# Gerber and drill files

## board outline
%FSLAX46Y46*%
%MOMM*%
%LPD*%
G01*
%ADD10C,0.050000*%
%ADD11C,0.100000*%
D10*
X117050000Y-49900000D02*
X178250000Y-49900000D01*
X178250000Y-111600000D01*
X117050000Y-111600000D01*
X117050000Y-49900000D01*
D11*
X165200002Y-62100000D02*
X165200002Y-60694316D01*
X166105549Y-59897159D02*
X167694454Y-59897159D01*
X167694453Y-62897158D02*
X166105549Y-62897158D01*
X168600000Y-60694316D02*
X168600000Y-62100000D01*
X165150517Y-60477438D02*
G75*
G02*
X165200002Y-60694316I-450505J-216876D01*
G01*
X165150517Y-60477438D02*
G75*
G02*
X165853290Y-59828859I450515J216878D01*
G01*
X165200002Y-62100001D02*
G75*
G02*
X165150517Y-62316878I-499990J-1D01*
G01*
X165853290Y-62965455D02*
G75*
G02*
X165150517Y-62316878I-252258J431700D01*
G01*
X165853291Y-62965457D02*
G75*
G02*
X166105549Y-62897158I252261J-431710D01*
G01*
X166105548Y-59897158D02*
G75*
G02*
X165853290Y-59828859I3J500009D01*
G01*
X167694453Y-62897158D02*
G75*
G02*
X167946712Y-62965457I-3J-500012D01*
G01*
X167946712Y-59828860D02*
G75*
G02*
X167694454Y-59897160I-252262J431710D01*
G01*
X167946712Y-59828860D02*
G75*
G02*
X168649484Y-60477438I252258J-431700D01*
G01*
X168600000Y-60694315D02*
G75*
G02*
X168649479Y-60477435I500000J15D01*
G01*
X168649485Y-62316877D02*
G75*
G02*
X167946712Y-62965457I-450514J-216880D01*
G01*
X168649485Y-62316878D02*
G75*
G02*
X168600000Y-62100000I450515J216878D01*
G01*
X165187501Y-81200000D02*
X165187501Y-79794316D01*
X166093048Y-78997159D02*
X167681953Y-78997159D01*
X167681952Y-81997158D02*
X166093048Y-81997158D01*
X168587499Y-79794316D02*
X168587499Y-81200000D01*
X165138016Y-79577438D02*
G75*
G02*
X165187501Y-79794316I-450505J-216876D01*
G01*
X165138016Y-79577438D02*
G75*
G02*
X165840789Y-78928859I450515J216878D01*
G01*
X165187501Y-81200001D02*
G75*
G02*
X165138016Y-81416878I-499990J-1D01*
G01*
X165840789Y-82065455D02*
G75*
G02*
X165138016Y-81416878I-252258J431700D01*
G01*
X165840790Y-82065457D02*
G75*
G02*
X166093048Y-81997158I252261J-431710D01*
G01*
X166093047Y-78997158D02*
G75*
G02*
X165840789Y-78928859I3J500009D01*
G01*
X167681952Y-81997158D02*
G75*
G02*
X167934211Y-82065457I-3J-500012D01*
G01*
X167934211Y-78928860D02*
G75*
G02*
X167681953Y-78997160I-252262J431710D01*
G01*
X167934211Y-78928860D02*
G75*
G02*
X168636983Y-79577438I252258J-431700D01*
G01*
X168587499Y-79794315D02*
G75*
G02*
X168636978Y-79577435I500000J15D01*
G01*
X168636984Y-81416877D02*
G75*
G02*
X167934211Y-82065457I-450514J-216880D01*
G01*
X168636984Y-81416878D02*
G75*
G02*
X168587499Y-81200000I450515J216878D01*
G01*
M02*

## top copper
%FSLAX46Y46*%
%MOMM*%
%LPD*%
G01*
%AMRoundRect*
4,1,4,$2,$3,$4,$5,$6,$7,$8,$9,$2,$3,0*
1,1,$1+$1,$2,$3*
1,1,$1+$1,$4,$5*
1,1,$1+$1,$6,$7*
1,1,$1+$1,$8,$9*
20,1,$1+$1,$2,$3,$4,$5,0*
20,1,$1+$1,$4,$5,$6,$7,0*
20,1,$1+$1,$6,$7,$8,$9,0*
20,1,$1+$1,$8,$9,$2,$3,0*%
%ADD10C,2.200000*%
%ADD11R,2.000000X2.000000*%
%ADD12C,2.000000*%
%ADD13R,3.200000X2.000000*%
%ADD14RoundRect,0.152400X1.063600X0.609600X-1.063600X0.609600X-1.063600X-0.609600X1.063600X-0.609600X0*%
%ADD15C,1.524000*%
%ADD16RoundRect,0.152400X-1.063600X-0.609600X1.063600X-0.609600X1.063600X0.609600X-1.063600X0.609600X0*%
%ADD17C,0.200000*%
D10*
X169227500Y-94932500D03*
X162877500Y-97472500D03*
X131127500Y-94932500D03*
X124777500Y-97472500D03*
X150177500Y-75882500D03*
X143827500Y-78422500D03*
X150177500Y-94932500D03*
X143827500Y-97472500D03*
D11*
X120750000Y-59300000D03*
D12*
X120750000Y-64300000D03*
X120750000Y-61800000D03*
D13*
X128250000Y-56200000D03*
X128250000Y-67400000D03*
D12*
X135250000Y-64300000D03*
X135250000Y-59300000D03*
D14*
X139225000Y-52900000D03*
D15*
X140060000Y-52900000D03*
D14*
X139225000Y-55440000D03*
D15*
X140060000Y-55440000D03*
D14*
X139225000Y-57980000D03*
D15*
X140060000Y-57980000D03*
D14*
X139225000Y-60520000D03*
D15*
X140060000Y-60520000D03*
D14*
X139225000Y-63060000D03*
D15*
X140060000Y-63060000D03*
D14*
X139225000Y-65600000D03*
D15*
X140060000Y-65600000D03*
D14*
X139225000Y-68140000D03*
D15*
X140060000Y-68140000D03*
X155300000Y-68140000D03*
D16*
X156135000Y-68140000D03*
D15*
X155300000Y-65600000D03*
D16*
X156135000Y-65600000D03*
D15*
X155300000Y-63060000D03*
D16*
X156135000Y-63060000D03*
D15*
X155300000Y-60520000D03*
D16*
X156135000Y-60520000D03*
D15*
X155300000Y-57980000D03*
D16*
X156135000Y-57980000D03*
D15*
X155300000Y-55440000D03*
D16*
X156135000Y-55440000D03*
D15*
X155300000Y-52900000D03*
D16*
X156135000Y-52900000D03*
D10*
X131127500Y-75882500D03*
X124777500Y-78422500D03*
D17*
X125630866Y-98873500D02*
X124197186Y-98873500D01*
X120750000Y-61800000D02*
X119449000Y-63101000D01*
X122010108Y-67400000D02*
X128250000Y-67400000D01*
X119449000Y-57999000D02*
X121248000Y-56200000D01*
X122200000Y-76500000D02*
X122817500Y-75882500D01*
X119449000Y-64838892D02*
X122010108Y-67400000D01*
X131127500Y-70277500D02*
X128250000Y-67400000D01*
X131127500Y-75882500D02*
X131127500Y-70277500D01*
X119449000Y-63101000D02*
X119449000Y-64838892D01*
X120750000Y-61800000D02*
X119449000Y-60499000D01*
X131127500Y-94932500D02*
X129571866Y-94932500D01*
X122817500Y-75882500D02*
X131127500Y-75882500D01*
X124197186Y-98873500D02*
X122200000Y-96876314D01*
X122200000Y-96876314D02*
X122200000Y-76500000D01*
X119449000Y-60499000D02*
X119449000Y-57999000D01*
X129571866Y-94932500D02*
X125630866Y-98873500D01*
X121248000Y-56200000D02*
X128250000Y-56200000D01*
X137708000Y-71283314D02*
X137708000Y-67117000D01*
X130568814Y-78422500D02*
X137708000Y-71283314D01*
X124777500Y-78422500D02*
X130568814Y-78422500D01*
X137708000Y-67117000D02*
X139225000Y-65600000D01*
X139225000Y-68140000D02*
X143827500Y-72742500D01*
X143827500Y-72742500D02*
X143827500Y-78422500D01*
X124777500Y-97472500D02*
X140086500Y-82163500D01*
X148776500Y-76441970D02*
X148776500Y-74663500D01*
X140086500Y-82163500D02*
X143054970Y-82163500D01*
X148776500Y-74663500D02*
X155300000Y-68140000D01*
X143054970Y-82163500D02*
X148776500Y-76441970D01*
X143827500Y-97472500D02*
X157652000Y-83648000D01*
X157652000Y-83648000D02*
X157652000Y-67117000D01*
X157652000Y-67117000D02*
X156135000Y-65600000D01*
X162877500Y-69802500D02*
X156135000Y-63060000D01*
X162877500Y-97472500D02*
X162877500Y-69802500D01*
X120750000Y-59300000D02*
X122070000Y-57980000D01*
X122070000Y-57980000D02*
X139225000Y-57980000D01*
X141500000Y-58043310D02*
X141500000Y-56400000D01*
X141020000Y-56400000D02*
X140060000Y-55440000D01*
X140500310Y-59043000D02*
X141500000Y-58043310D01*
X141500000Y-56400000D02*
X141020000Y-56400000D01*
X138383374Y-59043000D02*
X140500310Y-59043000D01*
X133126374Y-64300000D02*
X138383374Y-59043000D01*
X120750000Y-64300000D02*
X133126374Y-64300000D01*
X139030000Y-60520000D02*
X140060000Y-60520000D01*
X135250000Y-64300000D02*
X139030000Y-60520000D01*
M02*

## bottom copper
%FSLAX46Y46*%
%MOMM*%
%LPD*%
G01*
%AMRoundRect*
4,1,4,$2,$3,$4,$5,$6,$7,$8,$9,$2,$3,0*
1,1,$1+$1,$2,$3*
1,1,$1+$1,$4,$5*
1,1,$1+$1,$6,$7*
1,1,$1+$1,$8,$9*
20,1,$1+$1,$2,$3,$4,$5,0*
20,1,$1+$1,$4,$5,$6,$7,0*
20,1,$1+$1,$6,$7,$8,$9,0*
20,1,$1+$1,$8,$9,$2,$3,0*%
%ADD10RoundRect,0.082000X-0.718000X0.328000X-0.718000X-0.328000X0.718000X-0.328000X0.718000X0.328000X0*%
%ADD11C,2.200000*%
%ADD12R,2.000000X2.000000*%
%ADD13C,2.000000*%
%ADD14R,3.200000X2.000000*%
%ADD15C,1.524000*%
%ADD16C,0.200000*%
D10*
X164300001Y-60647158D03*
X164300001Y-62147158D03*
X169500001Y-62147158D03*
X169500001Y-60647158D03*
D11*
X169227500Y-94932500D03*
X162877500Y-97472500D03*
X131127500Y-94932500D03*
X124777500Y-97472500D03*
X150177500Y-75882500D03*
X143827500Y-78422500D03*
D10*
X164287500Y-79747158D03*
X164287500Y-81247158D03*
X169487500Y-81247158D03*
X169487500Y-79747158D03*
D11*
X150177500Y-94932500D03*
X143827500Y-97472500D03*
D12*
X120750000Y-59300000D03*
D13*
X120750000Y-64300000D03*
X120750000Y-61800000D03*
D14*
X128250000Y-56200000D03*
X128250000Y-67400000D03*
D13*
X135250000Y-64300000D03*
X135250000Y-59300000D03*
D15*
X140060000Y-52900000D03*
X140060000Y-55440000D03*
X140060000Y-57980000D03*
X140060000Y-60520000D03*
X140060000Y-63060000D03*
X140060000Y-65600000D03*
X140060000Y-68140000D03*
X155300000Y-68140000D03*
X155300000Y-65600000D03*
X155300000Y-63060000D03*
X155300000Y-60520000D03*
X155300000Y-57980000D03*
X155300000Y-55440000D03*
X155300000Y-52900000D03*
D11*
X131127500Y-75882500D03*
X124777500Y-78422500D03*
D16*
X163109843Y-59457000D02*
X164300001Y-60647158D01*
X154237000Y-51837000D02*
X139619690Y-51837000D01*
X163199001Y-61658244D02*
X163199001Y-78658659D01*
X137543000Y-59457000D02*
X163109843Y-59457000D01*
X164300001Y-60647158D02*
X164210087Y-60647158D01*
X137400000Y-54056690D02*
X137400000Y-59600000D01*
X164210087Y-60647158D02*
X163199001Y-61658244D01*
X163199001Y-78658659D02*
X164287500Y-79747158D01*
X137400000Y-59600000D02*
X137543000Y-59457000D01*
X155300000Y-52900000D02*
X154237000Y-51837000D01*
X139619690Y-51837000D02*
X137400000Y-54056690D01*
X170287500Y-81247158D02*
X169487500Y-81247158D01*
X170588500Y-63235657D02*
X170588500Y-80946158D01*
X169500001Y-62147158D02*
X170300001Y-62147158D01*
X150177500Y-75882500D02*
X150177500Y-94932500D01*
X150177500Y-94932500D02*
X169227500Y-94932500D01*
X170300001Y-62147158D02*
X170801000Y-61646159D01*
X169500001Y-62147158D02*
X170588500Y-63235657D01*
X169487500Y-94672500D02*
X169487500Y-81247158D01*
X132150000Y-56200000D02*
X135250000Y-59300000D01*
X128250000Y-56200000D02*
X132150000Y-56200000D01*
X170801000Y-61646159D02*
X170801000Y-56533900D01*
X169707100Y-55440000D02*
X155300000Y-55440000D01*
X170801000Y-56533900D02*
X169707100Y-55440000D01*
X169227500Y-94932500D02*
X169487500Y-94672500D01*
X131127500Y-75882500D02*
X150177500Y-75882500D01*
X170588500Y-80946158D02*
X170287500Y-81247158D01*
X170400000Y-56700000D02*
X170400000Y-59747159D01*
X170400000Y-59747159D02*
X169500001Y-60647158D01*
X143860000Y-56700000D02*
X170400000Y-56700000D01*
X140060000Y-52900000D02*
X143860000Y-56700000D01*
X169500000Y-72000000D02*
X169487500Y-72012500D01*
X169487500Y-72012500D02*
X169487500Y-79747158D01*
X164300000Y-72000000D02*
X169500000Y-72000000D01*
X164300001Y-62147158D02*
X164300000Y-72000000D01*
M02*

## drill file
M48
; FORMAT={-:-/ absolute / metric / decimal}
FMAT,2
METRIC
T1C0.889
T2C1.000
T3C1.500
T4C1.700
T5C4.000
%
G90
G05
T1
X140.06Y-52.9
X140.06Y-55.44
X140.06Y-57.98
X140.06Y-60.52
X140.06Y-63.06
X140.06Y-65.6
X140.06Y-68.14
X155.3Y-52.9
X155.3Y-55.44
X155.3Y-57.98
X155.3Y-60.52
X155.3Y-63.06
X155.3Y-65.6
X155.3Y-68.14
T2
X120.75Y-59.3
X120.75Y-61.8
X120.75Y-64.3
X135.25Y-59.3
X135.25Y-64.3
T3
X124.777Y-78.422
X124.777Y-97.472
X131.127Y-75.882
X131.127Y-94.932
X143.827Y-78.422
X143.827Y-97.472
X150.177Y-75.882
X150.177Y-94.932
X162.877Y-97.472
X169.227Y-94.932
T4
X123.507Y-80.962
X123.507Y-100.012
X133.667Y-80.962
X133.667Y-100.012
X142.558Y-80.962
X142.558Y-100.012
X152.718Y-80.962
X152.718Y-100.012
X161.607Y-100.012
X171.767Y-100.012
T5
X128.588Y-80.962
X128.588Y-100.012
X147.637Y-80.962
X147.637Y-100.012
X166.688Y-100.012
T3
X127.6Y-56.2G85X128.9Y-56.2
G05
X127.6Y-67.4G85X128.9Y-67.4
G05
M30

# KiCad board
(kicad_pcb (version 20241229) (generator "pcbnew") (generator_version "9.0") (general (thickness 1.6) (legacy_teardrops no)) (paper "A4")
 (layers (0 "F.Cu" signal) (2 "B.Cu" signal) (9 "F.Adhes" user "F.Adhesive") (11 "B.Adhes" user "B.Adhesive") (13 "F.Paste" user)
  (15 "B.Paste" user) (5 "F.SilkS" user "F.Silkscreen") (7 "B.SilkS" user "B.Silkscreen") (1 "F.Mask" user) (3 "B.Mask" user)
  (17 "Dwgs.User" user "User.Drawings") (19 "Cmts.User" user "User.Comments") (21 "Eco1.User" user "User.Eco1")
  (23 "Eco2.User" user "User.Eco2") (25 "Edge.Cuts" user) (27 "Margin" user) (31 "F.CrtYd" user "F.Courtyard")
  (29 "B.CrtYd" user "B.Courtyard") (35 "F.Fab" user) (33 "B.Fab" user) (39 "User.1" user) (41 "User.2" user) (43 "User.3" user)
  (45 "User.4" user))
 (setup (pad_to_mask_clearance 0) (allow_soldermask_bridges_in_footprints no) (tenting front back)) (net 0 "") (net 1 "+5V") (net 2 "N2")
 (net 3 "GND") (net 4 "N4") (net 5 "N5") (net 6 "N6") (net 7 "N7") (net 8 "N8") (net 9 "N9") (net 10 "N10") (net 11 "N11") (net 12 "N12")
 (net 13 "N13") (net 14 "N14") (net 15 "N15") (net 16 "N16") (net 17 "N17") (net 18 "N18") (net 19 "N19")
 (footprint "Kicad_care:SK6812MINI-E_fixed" (layer "F.Cu") (at 166.9 61.5)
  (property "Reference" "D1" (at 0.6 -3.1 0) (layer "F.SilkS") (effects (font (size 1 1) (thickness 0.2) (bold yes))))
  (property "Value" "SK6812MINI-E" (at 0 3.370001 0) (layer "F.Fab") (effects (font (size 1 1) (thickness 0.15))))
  (fp_line (start -1.699998 0.6) (end -1.699998 -0.805684) (stroke (width 0.1) (type solid)) (layer "Edge.Cuts"))
  (fp_line (start -0.794451 -1.602841) (end 0.794454 -1.602841) (stroke (width 0.1) (type solid)) (layer "Edge.Cuts"))
  (fp_line (start 0.794453 1.397158) (end -0.794451 1.397158) (stroke (width 0.1) (type solid)) (layer "Edge.Cuts"))
  (fp_line (start 1.7 -0.805684) (end 1.7 0.6) (stroke (width 0.1) (type solid)) (layer "Edge.Cuts"))
  (fp_arc (start -1.749483 -1.022562) (mid -1.712526 -0.91691) (end -1.699998 -0.805684) (stroke (width 0.1) (type solid))
   (layer "Edge.Cuts"))
  (fp_arc (start -1.749483 -1.022562) (mid -1.63807 -1.606877) (end -1.04671 -1.671141) (stroke (width 0.1) (type solid))
   (layer "Edge.Cuts"))
  (fp_arc (start -1.699998 0.600001) (mid -1.712526 0.711226) (end -1.749483 0.816878) (stroke (width 0.1) (type solid)) (layer "Edge.Cuts"))
  (fp_arc (start -1.04671 1.465455) (mid -1.638069 1.401192) (end -1.749483 0.816878) (stroke (width 0.1) (type solid)) (layer "Edge.Cuts"))
  (fp_arc (start -1.046709 1.465457) (mid -0.925121 1.414535) (end -0.794451 1.397158) (stroke (width 0.1) (type solid)) (layer "Edge.Cuts"))
  (fp_arc (start -0.794452 -1.602842) (mid -0.925122 -1.620219) (end -1.04671 -1.671141) (stroke (width 0.1) (type solid))
   (layer "Edge.Cuts"))
  (fp_arc (start 0.794453 1.397158) (mid 0.925124 1.414535) (end 1.046712 1.465457) (stroke (width 0.1) (type solid)) (layer "Edge.Cuts"))
  (fp_arc (start 1.046712 -1.67114) (mid 0.925124 -1.620218) (end 0.794454 -1.602841) (stroke (width 0.1) (type solid)) (layer "Edge.Cuts"))
  (fp_arc (start 1.046712 -1.67114) (mid 1.638072 -1.606876) (end 1.749485 -1.022562) (stroke (width 0.1) (type solid)) (layer "Edge.Cuts"))
  (fp_arc (start 1.7 -0.805685) (mid 1.712528 -0.91691) (end 1.749485 -1.022562) (stroke (width 0.1) (type solid)) (layer "Edge.Cuts"))
  (fp_arc (start 1.749485 0.816877) (mid 1.638073 1.401193) (end 1.046712 1.465457) (stroke (width 0.1) (type solid)) (layer "Edge.Cuts"))
  (fp_arc (start 1.749485 0.816878) (mid 1.712528 0.711226) (end 1.7 0.6) (stroke (width 0.1) (type solid)) (layer "Edge.Cuts"))
  (pad "1" smd roundrect (at -2.599999 -0.852842 270) (size 0.82 1.6) (layers "B.Cu" "B.Mask" "B.Paste") (roundrect_rratio 0.1)
   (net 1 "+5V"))
  (pad "2" smd roundrect (at -2.599999 0.647158 270) (size 0.82 1.6) (layers "B.Cu" "B.Mask" "B.Paste") (roundrect_rratio 0.1) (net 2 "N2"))
  (pad "3" smd roundrect (at 2.600001 0.647158 270) (size 0.82 1.6) (layers "B.Cu" "B.Mask" "B.Paste") (roundrect_rratio 0.1) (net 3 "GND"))
  (pad "4" smd roundrect (at 2.600001 -0.852842 270) (size 0.82 1.6) (layers "B.Cu" "B.Mask" "B.Paste") (roundrect_rratio 0.1) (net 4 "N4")))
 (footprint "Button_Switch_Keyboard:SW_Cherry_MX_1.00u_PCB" (layer "F.Cu") (at 169.2275 94.9325)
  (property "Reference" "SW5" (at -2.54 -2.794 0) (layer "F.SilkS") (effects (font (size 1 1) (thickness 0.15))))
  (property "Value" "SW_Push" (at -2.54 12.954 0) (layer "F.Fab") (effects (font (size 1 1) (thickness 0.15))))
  (pad "" np_thru_hole circle (at -7.62 5.08) (size 1.7 1.7) (drill 1.7) (layers "*.Cu" "*.Mask"))
  (pad "" np_thru_hole circle (at -2.54 5.08) (size 4 4) (drill 4) (layers "*.Cu" "*.Mask"))
  (pad "" np_thru_hole circle (at 2.54 5.08) (size 1.7 1.7) (drill 1.7) (layers "*.Cu" "*.Mask"))
  (pad "1" thru_hole circle (at 0 0) (size 2.2 2.2) (drill 1.5) (layers "*.Cu" "*.Mask") (remove_unused_layers no) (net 3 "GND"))
  (pad "2" thru_hole circle (at -6.35 2.54) (size 2.2 2.2) (drill 1.5) (layers "*.Cu" "*.Mask") (remove_unused_layers no) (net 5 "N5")))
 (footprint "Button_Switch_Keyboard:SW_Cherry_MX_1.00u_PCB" (layer "F.Cu") (at 131.1275 94.9325)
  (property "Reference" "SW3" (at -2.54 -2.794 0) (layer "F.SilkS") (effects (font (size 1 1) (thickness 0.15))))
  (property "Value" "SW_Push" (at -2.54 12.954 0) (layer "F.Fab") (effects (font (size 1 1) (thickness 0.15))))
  (pad "" np_thru_hole circle (at -7.62 5.08) (size 1.7 1.7) (drill 1.7) (layers "*.Cu" "*.Mask"))
  (pad "" np_thru_hole circle (at -2.54 5.08) (size 4 4) (drill 4) (layers "*.Cu" "*.Mask"))
  (pad "" np_thru_hole circle (at 2.54 5.08) (size 1.7 1.7) (drill 1.7) (layers "*.Cu" "*.Mask"))
  (pad "1" thru_hole circle (at 0 0) (size 2.2 2.2) (drill 1.5) (layers "*.Cu" "*.Mask") (remove_unused_layers no) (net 3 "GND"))
  (pad "2" thru_hole circle (at -6.35 2.54) (size 2.2 2.2) (drill 1.5) (layers "*.Cu" "*.Mask") (remove_unused_layers no) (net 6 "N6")))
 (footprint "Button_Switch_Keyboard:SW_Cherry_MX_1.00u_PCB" (layer "F.Cu") (at 150.1775 75.8825)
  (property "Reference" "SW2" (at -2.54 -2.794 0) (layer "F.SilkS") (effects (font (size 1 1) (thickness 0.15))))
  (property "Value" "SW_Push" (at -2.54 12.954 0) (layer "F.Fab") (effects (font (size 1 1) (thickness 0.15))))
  (pad "" np_thru_hole circle (at -7.62 5.08) (size 1.7 1.7) (drill 1.7) (layers "*.Cu" "*.Mask"))
  (pad "" np_thru_hole circle (at -2.54 5.08) (size 4 4) (drill 4) (layers "*.Cu" "*.Mask"))
  (pad "" np_thru_hole circle (at 2.54 5.08) (size 1.7 1.7) (drill 1.7) (layers "*.Cu" "*.Mask"))
  (pad "1" thru_hole circle (at 0 0) (size 2.2 2.2) (drill 1.5) (layers "*.Cu" "*.Mask") (remove_unused_layers no) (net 3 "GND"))
  (pad "2" thru_hole circle (at -6.35 2.54) (size 2.2 2.2) (drill 1.5) (layers "*.Cu" "*.Mask") (remove_unused_layers no) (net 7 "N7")))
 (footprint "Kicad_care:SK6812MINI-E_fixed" (layer "F.Cu") (at 166.887499 80.6)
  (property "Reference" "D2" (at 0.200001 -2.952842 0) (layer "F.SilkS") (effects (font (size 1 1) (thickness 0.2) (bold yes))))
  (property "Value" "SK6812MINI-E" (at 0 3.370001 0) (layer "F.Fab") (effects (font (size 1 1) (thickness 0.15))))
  (fp_line (start -1.699998 0.6) (end -1.699998 -0.805684) (stroke (width 0.1) (type solid)) (layer "Edge.Cuts"))
  (fp_line (start -0.794451 -1.602841) (end 0.794454 -1.602841) (stroke (width 0.1) (type solid)) (layer "Edge.Cuts"))
  (fp_line (start 0.794453 1.397158) (end -0.794451 1.397158) (stroke (width 0.1) (type solid)) (layer "Edge.Cuts"))
  (fp_line (start 1.7 -0.805684) (end 1.7 0.6) (stroke (width 0.1) (type solid)) (layer "Edge.Cuts"))
  (fp_arc (start -1.749483 -1.022562) (mid -1.712526 -0.91691) (end -1.699998 -0.805684) (stroke (width 0.1) (type solid))
   (layer "Edge.Cuts"))
  (fp_arc (start -1.749483 -1.022562) (mid -1.63807 -1.606877) (end -1.04671 -1.671141) (stroke (width 0.1) (type solid))
   (layer "Edge.Cuts"))
  (fp_arc (start -1.699998 0.600001) (mid -1.712526 0.711226) (end -1.749483 0.816878) (stroke (width 0.1) (type solid)) (layer "Edge.Cuts"))
  (fp_arc (start -1.04671 1.465455) (mid -1.638069 1.401192) (end -1.749483 0.816878) (stroke (width 0.1) (type solid)) (layer "Edge.Cuts"))
  (fp_arc (start -1.046709 1.465457) (mid -0.925121 1.414535) (end -0.794451 1.397158) (stroke (width 0.1) (type solid)) (layer "Edge.Cuts"))
  (fp_arc (start -0.794452 -1.602842) (mid -0.925122 -1.620219) (end -1.04671 -1.671141) (stroke (width 0.1) (type solid))
   (layer "Edge.Cuts"))
  (fp_arc (start 0.794453 1.397158) (mid 0.925124 1.414535) (end 1.046712 1.465457) (stroke (width 0.1) (type solid)) (layer "Edge.Cuts"))
  (fp_arc (start 1.046712 -1.67114) (mid 0.925124 -1.620218) (end 0.794454 -1.602841) (stroke (width 0.1) (type solid)) (layer "Edge.Cuts"))
  (fp_arc (start 1.046712 -1.67114) (mid 1.638072 -1.606876) (end 1.749485 -1.022562) (stroke (width 0.1) (type solid)) (layer "Edge.Cuts"))
  (fp_arc (start 1.7 -0.805685) (mid 1.712528 -0.91691) (end 1.749485 -1.022562) (stroke (width 0.1) (type solid)) (layer "Edge.Cuts"))
  (fp_arc (start 1.749485 0.816877) (mid 1.638073 1.401193) (end 1.046712 1.465457) (stroke (width 0.1) (type solid)) (layer "Edge.Cuts"))
  (fp_arc (start 1.749485 0.816878) (mid 1.712528 0.711226) (end 1.7 0.6) (stroke (width 0.1) (type solid)) (layer "Edge.Cuts"))
  (pad "1" smd roundrect (at -2.599999 -0.852842 270) (size 0.82 1.6) (layers "B.Cu" "B.Mask" "B.Paste") (roundrect_rratio 0.1)
   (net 1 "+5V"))
  (pad "2" smd roundrect (at -2.599999 0.647158 270) (size 0.82 1.6) (layers "B.Cu" "B.Mask" "B.Paste") (roundrect_rratio 0.1) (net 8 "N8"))
  (pad "3" smd roundrect (at 2.600001 0.647158 270) (size 0.82 1.6) (layers "B.Cu" "B.Mask" "B.Paste") (roundrect_rratio 0.1) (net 3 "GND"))
  (pad "4" smd roundrect (at 2.600001 -0.852842 270) (size 0.82 1.6) (layers "B.Cu" "B.Mask" "B.Paste") (roundrect_rratio 0.1) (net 2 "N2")))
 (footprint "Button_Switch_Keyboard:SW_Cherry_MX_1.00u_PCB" (layer "F.Cu") (at 150.1775 94.9325)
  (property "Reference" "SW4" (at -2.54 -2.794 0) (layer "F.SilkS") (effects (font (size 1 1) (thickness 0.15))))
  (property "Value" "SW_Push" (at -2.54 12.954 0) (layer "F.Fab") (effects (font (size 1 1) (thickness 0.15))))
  (pad "" np_thru_hole circle (at -7.62 5.08) (size 1.7 1.7) (drill 1.7) (layers "*.Cu" "*.Mask"))
  (pad "" np_thru_hole circle (at -2.54 5.08) (size 4 4) (drill 4) (layers "*.Cu" "*.Mask"))
  (pad "" np_thru_hole circle (at 2.54 5.08) (size 1.7 1.7) (drill 1.7) (layers "*.Cu" "*.Mask"))
  (pad "1" thru_hole circle (at 0 0) (size 2.2 2.2) (drill 1.5) (layers "*.Cu" "*.Mask") (remove_unused_layers no) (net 3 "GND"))
  (pad "2" thru_hole circle (at -6.35 2.54) (size 2.2 2.2) (drill 1.5) (layers "*.Cu" "*.Mask") (remove_unused_layers no) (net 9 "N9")))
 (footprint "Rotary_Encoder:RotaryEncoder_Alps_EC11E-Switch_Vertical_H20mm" (layer "F.Cu") (at 120.75 59.3)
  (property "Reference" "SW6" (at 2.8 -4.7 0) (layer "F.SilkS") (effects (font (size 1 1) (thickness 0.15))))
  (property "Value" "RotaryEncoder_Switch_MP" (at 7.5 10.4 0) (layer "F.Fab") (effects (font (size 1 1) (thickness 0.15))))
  (pad "A" thru_hole rect (at 0 0) (size 2 2) (drill 1) (layers "*.Cu" "*.Mask") (remove_unused_layers no) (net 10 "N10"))
  (pad "B" thru_hole circle (at 0 5) (size 2 2) (drill 1) (layers "*.Cu" "*.Mask") (remove_unused_layers no) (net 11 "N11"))
  (pad "C" thru_hole circle (at 0 2.5) (size 2 2) (drill 1) (layers "*.Cu" "*.Mask") (remove_unused_layers no) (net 3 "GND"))
  (pad "MP" thru_hole rect (at 7.5 -3.1) (size 3.2 2) (drill oval 2.8 1.5) (layers "*.Cu" "*.Mask") (remove_unused_layers no) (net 3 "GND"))
  (pad "MP" thru_hole rect (at 7.5 8.1) (size 3.2 2) (drill oval 2.8 1.5) (layers "*.Cu" "*.Mask") (remove_unused_layers no) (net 3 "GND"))
  (pad "S1" thru_hole circle (at 14.5 5) (size 2 2) (drill 1) (layers "*.Cu" "*.Mask") (remove_unused_layers no) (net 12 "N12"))
  (pad "S2" thru_hole circle (at 14.5 0) (size 2 2) (drill 1) (layers "*.Cu" "*.Mask") (remove_unused_layers no) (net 3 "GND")))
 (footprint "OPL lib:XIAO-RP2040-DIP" (layer "F.Cu") (at 147.68 60.52)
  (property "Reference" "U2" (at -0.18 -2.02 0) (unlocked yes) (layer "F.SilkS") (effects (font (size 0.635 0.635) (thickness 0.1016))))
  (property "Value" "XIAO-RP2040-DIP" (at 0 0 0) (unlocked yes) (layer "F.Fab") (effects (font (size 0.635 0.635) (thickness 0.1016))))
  (pad "1" smd roundrect (at -8.455 -7.62 180) (size 2.432 1.524) (layers "F.Cu" "F.Mask") (roundrect_rratio 0.1) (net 4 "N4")
   (thermal_bridge_angle 45))
  (pad "1" thru_hole circle (at -7.62 -7.62 180) (size 1.524 1.524) (drill 0.889) (layers "*.Cu" "*.Mask") (remove_unused_layers no)
   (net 4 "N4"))
  (pad "2" smd roundrect (at -8.455 -5.08 180) (size 2.432 1.524) (layers "F.Cu" "F.Mask") (roundrect_rratio 0.1) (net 11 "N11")
   (thermal_bridge_angle 45))
  (pad "2" thru_hole circle (at -7.62 -5.08 180) (size 1.524 1.524) (drill 0.889) (layers "*.Cu" "*.Mask") (remove_unused_layers no)
   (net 11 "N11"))
  (pad "3" smd roundrect (at -8.455 -2.54 180) (size 2.432 1.524) (layers "F.Cu" "F.Mask") (roundrect_rratio 0.1) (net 10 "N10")
   (thermal_bridge_angle 45))
  (pad "3" thru_hole circle (at -7.62 -2.54 180) (size 1.524 1.524) (drill 0.889) (layers "*.Cu" "*.Mask") (remove_unused_layers no)
   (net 10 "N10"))
  (pad "4" smd roundrect (at -8.455 0 180) (size 2.432 1.524) (layers "F.Cu" "F.Mask") (roundrect_rratio 0.1) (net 12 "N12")
   (thermal_bridge_angle 45))
  (pad "4" thru_hole circle (at -7.62 0 180) (size 1.524 1.524) (drill 0.889) (layers "*.Cu" "*.Mask") (remove_unused_layers no)
   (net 12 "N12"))
  (pad "5" smd roundrect (at -8.455 2.54 180) (size 2.432 1.524) (layers "F.Cu" "F.Mask") (roundrect_rratio 0.1) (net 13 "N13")
   (thermal_bridge_angle 45))
  (pad "5" thru_hole circle (at -7.62 2.54 180) (size 1.524 1.524) (drill 0.889) (layers "*.Cu" "*.Mask") (remove_unused_layers no)
   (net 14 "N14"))
  (pad "6" smd roundrect (at -8.455 5.08 180) (size 2.432 1.524) (layers "F.Cu" "F.Mask") (roundrect_rratio 0.1) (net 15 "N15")
   (thermal_bridge_angle 45))
  (pad "6" thru_hole circle (at -7.62 5.08 180) (size 1.524 1.524) (drill 0.889) (layers "*.Cu" "*.Mask") (remove_unused_layers no)
   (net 15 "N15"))
  (pad "7" smd roundrect (at -8.455 7.62 180) (size 2.432 1.524) (layers "F.Cu" "F.Mask") (roundrect_rratio 0.1) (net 7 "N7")
   (thermal_bridge_angle 45))
  (pad "7" thru_hole circle (at -7.62 7.62 180) (size 1.524 1.524) (drill 0.889) (layers "*.Cu" "*.Mask") (remove_unused_layers no)
   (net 7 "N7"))
  (pad "8" thru_hole circle (at 7.62 7.62) (size 1.524 1.524) (drill 0.889) (layers "*.Cu" "*.Mask") (remove_unused_layers no) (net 6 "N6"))
  (pad "8" smd roundrect (at 8.455 7.62) (size 2.432 1.524) (layers "F.Cu" "F.Mask") (roundrect_rratio 0.1) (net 6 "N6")
   (thermal_bridge_angle 45))
  (pad "9" thru_hole circle (at 7.62 5.08) (size 1.524 1.524) (drill 0.889) (layers "*.Cu" "*.Mask") (remove_unused_layers no) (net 9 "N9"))
  (pad "9" smd roundrect (at 8.455 5.08) (size 2.432 1.524) (layers "F.Cu" "F.Mask") (roundrect_rratio 0.1) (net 9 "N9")
   (thermal_bridge_angle 45))
  (pad "10" thru_hole circle (at 7.62 2.54) (size 1.524 1.524) (drill 0.889) (layers "*.Cu" "*.Mask") (remove_unused_layers no) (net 5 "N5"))
  (pad "10" smd roundrect (at 8.455 2.54) (size 2.432 1.524) (layers "F.Cu" "F.Mask") (roundrect_rratio 0.1) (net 5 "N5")
   (thermal_bridge_angle 45))
  (pad "11" thru_hole circle (at 7.62 0) (size 1.524 1.524) (drill 0.889) (layers "*.Cu" "*.Mask") (remove_unused_layers no) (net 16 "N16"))
  (pad "11" smd roundrect (at 8.455 0) (size 2.432 1.524) (layers "F.Cu" "F.Mask") (roundrect_rratio 0.1) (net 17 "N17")
   (thermal_bridge_angle 45))
  (pad "12" thru_hole circle (at 7.62 -2.54) (size 1.524 1.524) (drill 0.889) (layers "*.Cu" "*.Mask") (remove_unused_layers no)
   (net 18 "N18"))
  (pad "12" smd roundrect (at 8.455 -2.54) (size 2.432 1.524) (layers "F.Cu" "F.Mask") (roundrect_rratio 0.1) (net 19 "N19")
   (thermal_bridge_angle 45))
  (pad "13" thru_hole circle (at 7.62 -5.08) (size 1.524 1.524) (drill 0.889) (layers "*.Cu" "*.Mask") (remove_unused_layers no)
   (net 3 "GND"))
  (pad "13" smd roundrect (at 8.455 -5.08) (size 2.432 1.524) (layers "F.Cu" "F.Mask") (roundrect_rratio 0.1) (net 3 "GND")
   (thermal_bridge_angle 45))
  (pad "14" thru_hole circle (at 7.62 -7.62) (size 1.524 1.524) (drill 0.889) (layers "*.Cu" "*.Mask") (remove_unused_layers no)
   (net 1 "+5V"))
  (pad "14" smd roundrect (at 8.455 -7.62) (size 2.432 1.524) (layers "F.Cu" "F.Mask") (roundrect_rratio 0.1) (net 1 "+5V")
   (thermal_bridge_angle 45)))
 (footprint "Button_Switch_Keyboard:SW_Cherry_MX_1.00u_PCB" (layer "F.Cu") (at 131.1275 75.8825)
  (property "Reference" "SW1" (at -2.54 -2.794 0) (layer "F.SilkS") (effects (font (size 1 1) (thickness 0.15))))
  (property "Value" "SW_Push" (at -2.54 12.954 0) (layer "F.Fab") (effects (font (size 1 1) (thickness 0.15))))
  (pad "" np_thru_hole circle (at -7.62 5.08) (size 1.7 1.7) (drill 1.7) (layers "*.Cu" "*.Mask"))
  (pad "" np_thru_hole circle (at -2.54 5.08) (size 4 4) (drill 4) (layers "*.Cu" "*.Mask"))
  (pad "" np_thru_hole circle (at 2.54 5.08) (size 1.7 1.7) (drill 1.7) (layers "*.Cu" "*.Mask"))
  (pad "1" thru_hole circle (at 0 0) (size 2.2 2.2) (drill 1.5) (layers "*.Cu" "*.Mask") (remove_unused_layers no) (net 3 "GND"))
  (pad "2" thru_hole circle (at -6.35 2.54) (size 2.2 2.2) (drill 1.5) (layers "*.Cu" "*.Mask") (remove_unused_layers no) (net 15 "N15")))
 (gr_rect (start 117.05 49.9) (end 178.25 111.6) (stroke (width 0.05) (type default)) (fill no) (layer "Edge.Cuts"))
 (segment (start 163.109843 59.457) (end 164.300001 60.647158) (width 0.2) (layer "B.Cu") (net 1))
 (segment (start 154.237 51.837) (end 139.61969 51.837) (width 0.2) (layer "B.Cu") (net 1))
 (segment (start 163.199001 61.658244) (end 163.199001 78.658659) (width 0.2) (layer "B.Cu") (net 1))
 (segment (start 137.543 59.457) (end 163.109843 59.457) (width 0.2) (layer "B.Cu") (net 1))
 (segment (start 164.300001 60.647158) (end 164.210087 60.647158) (width 0.2) (layer "B.Cu") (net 1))
 (segment (start 137.4 54.05669) (end 137.4 59.6) (width 0.2) (layer "B.Cu") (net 1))
 (segment (start 164.210087 60.647158) (end 163.199001 61.658244) (width 0.2) (layer "B.Cu") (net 1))
 (segment (start 163.199001 78.658659) (end 164.2875 79.747158) (width 0.2) (layer "B.Cu") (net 1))
 (segment (start 137.4 59.6) (end 137.543 59.457) (width 0.2) (layer "B.Cu") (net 1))
 (segment (start 155.3 52.9) (end 154.237 51.837) (width 0.2) (layer "B.Cu") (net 1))
 (segment (start 139.61969 51.837) (end 137.4 54.05669) (width 0.2) (layer "B.Cu") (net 1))
 (segment (start 125.630866 98.8735) (end 124.197186 98.8735) (width 0.2) (layer "F.Cu") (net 3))
 (segment (start 120.75 61.8) (end 119.449 63.101) (width 0.2) (layer "F.Cu") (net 3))
 (segment (start 122.010108 67.4) (end 128.25 67.4) (width 0.2) (layer "F.Cu") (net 3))
 (segment (start 119.449 57.999) (end 121.248 56.2) (width 0.2) (layer "F.Cu") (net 3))
 (segment (start 122.2 76.5) (end 122.8175 75.8825) (width 0.2) (layer "F.Cu") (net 3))
 (segment (start 119.449 64.838892) (end 122.010108 67.4) (width 0.2) (layer "F.Cu") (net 3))
 (segment (start 131.1275 70.2775) (end 128.25 67.4) (width 0.2) (layer "F.Cu") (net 3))
 (segment (start 131.1275 75.8825) (end 131.1275 70.2775) (width 0.2) (layer "F.Cu") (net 3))
 (segment (start 119.449 63.101) (end 119.449 64.838892) (width 0.2) (layer "F.Cu") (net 3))
 (segment (start 120.75 61.8) (end 119.449 60.499) (width 0.2) (layer "F.Cu") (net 3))
 (segment (start 131.1275 94.9325) (end 129.571866 94.9325) (width 0.2) (layer "F.Cu") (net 3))
 (segment (start 122.8175 75.8825) (end 131.1275 75.8825) (width 0.2) (layer "F.Cu") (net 3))
 (segment (start 124.197186 98.8735) (end 122.2 96.876314) (width 0.2) (layer "F.Cu") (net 3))
 (segment (start 122.2 96.876314) (end 122.2 76.5) (width 0.2) (layer "F.Cu") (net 3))
 (segment (start 119.449 60.499) (end 119.449 57.999) (width 0.2) (layer "F.Cu") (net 3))
 (segment (start 129.571866 94.9325) (end 125.630866 98.8735) (width 0.2) (layer "F.Cu") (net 3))
 (segment (start 121.248 56.2) (end 128.25 56.2) (width 0.2) (layer "F.Cu") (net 3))
 (segment (start 170.2875 81.247158) (end 169.4875 81.247158) (width 0.2) (layer "B.Cu") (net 3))
 (segment (start 170.5885 63.235657) (end 170.5885 80.946158) (width 0.2) (layer "B.Cu") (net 3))
 (segment (start 169.500001 62.147158) (end 170.300001 62.147158) (width 0.2) (layer "B.Cu") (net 3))
 (segment (start 150.1775 75.8825) (end 150.1775 94.9325) (width 0.2) (layer "B.Cu") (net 3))
 (segment (start 150.1775 94.9325) (end 169.2275 94.9325) (width 0.2) (layer "B.Cu") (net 3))
 (segment (start 170.300001 62.147158) (end 170.801 61.646159) (width 0.2) (layer "B.Cu") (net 3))
 (segment (start 169.500001 62.147158) (end 170.5885 63.235657) (width 0.2) (layer "B.Cu") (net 3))
 (segment (start 169.4875 94.6725) (end 169.4875 81.247158) (width 0.2) (layer "B.Cu") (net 3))
 (segment (start 132.15 56.2) (end 135.25 59.3) (width 0.2) (layer "B.Cu") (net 3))
 (segment (start 128.25 56.2) (end 132.15 56.2) (width 0.2) (layer "B.Cu") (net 3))
 (segment (start 170.801 61.646159) (end 170.801 56.5339) (width 0.2) (layer "B.Cu") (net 3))
 (segment (start 169.7071 55.44) (end 155.3 55.44) (width 0.2) (layer "B.Cu") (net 3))
 (segment (start 170.801 56.5339) (end 169.7071 55.44) (width 0.2) (layer "B.Cu") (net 3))
 (segment (start 169.2275 94.9325) (end 169.4875 94.6725) (width 0.2) (layer "B.Cu") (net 3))
 (segment (start 131.1275 75.8825) (end 150.1775 75.8825) (width 0.2) (layer "B.Cu") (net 3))
 (segment (start 170.5885 80.946158) (end 170.2875 81.247158) (width 0.2) (layer "B.Cu") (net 3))
 (segment (start 170.4 56.7) (end 170.4 59.747159) (width 0.2) (layer "B.Cu") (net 4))
 (segment (start 170.4 59.747159) (end 169.500001 60.647158) (width 0.2) (layer "B.Cu") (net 4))
 (segment (start 143.86 56.7) (end 170.4 56.7) (width 0.2) (layer "B.Cu") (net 4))
 (segment (start 140.06 52.9) (end 143.86 56.7) (width 0.2) (layer "B.Cu") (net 4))
 (segment (start 169.5 72) (end 169.4875 72.0125) (width 0.2) (layer "B.Cu") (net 2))
 (segment (start 169.4875 72.0125) (end 169.4875 79.747158) (width 0.2) (layer "B.Cu") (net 2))
 (segment (start 164.3 72) (end 169.5 72) (width 0.2) (layer "B.Cu") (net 2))
 (segment (start 164.300001 62.147158) (end 164.3 72) (width 0.2) (layer "B.Cu") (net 2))
 (segment (start 137.708 71.283314) (end 137.708 67.117) (width 0.2) (layer "F.Cu") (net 15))
 (segment (start 130.568814 78.4225) (end 137.708 71.283314) (width 0.2) (layer "F.Cu") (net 15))
 (segment (start 124.7775 78.4225) (end 130.568814 78.4225) (width 0.2) (layer "F.Cu") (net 15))
 (segment (start 137.708 67.117) (end 139.225 65.6) (width 0.2) (layer "F.Cu") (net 15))
 (segment (start 139.225 68.14) (end 143.8275 72.7425) (width 0.2) (layer "F.Cu") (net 7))
 (segment (start 143.8275 72.7425) (end 143.8275 78.4225) (width 0.2) (layer "F.Cu") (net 7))
 (segment (start 124.7775 97.4725) (end 140.0865 82.1635) (width 0.2) (layer "F.Cu") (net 6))
 (segment (start 148.7765 76.44197) (end 148.7765 74.6635) (width 0.2) (layer "F.Cu") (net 6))
 (segment (start 140.0865 82.1635) (end 143.05497 82.1635) (width 0.2) (layer "F.Cu") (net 6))
 (segment (start 148.7765 74.6635) (end 155.3 68.14) (width 0.2) (layer "F.Cu") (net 6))
 (segment (start 143.05497 82.1635) (end 148.7765 76.44197) (width 0.2) (layer "F.Cu") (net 6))
 (segment (start 143.8275 97.4725) (end 157.652 83.648) (width 0.2) (layer "F.Cu") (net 9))
 (segment (start 157.652 83.648) (end 157.652 67.117) (width 0.2) (layer "F.Cu") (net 9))
 (segment (start 157.652 67.117) (end 156.135 65.6) (width 0.2) (layer "F.Cu") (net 9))
 (segment (start 162.8775 69.8025) (end 156.135 63.06) (width 0.2) (layer "F.Cu") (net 5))
 (segment (start 162.8775 97.4725) (end 162.8775 69.8025) (width 0.2) (layer "F.Cu") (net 5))
 (segment (start 120.75 59.3) (end 122.07 57.98) (width 0.2) (layer "F.Cu") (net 10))
 (segment (start 122.07 57.98) (end 139.225 57.98) (width 0.2) (layer "F.Cu") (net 10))
 (segment (start 141.5 58.04331) (end 141.5 56.4) (width 0.2) (layer "F.Cu") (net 11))
 (segment (start 141.02 56.4) (end 140.06 55.44) (width 0.2) (layer "F.Cu") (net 11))
 (segment (start 140.50031 59.043) (end 141.5 58.04331) (width 0.2) (layer "F.Cu") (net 11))
 (segment (start 141.5 56.4) (end 141.02 56.4) (width 0.2) (layer "F.Cu") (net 11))
 (segment (start 138.383374 59.043) (end 140.50031 59.043) (width 0.2) (layer "F.Cu") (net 11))
 (segment (start 133.126374 64.3) (end 138.383374 59.043) (width 0.2) (layer "F.Cu") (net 11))
 (segment (start 120.75 64.3) (end 133.126374 64.3) (width 0.2) (layer "F.Cu") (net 11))
 (segment (start 139.03 60.52) (end 140.06 60.52) (width 0.2) (layer "F.Cu") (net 12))
 (segment (start 135.25 64.3) (end 139.03 60.52) (width 0.2) (layer "F.Cu") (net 12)))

